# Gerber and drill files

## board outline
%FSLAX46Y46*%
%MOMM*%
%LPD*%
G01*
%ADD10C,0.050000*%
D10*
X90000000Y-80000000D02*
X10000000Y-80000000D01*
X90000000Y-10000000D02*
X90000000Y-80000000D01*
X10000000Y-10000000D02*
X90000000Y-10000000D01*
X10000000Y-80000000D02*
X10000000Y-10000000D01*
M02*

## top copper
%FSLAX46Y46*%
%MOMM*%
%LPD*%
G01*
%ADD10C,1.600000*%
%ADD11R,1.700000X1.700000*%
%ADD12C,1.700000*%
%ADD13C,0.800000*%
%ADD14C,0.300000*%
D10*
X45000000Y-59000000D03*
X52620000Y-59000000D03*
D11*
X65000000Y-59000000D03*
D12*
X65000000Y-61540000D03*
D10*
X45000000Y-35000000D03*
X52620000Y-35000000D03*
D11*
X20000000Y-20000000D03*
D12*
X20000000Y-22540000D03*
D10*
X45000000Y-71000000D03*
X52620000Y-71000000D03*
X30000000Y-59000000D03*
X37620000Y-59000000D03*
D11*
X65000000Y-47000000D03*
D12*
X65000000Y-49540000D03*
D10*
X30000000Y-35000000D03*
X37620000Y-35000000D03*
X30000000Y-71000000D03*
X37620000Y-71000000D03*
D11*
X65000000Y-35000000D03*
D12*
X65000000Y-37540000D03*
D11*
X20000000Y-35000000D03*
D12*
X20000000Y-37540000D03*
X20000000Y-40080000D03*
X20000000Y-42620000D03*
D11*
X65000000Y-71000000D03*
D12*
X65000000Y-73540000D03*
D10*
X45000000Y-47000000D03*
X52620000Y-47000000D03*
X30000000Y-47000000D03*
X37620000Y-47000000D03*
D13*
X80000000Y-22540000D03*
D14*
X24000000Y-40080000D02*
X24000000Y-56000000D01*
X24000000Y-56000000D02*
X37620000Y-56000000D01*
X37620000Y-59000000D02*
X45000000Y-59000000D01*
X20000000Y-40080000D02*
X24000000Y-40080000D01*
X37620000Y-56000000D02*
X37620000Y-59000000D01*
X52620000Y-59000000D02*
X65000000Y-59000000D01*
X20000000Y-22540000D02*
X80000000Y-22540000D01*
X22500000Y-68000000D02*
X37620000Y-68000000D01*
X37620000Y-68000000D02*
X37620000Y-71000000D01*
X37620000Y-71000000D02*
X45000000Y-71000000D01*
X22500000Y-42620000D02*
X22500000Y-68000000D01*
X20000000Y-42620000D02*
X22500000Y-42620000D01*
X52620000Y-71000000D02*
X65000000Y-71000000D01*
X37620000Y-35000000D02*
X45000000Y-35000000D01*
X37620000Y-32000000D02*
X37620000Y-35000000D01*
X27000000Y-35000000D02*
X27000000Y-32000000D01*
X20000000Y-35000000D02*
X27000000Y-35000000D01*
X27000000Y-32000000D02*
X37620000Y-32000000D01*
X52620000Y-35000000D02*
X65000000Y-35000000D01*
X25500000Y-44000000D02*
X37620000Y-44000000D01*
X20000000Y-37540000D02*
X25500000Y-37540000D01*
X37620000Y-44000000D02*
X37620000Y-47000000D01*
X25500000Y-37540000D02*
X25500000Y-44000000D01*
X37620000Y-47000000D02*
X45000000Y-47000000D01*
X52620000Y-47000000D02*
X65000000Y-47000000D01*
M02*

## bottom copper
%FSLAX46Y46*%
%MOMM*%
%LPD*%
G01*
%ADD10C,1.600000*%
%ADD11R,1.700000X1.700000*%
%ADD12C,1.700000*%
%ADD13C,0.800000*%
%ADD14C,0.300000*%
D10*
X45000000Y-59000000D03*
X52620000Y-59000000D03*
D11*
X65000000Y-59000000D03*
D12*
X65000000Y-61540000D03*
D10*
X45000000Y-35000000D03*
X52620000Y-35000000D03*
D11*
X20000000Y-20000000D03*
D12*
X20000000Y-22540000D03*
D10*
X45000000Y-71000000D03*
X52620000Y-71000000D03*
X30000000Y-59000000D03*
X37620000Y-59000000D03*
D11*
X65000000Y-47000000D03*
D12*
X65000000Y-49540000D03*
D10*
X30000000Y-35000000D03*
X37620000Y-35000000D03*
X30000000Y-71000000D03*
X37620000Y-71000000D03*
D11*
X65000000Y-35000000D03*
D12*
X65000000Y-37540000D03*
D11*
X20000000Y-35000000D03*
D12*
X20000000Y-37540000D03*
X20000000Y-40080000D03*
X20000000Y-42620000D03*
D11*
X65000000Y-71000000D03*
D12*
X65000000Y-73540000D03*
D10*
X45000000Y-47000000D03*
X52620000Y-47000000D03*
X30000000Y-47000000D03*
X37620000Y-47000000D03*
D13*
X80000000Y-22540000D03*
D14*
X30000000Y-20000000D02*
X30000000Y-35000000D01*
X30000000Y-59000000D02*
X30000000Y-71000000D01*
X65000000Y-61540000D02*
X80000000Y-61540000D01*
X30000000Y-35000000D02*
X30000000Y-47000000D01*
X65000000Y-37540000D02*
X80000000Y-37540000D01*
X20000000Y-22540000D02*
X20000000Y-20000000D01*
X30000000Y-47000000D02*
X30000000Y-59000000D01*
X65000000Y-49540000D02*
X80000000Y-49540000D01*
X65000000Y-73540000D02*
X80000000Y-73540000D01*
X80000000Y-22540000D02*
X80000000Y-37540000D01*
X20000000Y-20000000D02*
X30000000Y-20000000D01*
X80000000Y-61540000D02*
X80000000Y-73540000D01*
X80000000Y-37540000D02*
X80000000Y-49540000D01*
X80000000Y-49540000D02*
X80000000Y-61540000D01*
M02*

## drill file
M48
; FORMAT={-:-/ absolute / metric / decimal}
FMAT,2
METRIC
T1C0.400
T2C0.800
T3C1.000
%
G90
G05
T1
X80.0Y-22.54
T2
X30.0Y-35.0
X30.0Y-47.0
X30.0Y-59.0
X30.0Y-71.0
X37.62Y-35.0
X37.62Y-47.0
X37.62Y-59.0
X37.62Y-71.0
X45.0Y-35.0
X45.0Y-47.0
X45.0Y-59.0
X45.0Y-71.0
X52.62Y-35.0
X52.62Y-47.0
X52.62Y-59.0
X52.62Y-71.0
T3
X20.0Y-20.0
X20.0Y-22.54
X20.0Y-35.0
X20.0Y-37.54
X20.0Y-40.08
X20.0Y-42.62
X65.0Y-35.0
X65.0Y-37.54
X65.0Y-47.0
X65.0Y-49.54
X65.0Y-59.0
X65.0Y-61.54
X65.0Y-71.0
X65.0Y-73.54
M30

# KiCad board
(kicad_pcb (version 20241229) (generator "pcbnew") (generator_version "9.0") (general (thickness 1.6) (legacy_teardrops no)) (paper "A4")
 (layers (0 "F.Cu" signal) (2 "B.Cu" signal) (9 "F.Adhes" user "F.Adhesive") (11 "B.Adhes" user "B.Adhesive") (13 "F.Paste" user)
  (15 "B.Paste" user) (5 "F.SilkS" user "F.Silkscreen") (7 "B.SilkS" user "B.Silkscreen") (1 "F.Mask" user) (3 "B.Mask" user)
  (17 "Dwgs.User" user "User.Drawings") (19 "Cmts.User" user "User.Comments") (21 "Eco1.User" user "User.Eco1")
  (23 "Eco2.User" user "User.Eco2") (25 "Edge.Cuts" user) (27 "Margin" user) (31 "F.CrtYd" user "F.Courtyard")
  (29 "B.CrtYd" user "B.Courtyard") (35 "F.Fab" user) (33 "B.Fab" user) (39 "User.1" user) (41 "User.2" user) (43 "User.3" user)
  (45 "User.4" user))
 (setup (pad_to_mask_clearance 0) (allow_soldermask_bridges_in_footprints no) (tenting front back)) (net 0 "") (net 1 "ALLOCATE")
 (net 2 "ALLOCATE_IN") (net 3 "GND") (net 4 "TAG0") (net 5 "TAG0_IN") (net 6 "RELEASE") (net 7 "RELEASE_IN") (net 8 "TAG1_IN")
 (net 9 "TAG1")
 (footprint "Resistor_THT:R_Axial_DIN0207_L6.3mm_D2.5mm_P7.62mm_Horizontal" (layer "F.Cu") (at 45 59)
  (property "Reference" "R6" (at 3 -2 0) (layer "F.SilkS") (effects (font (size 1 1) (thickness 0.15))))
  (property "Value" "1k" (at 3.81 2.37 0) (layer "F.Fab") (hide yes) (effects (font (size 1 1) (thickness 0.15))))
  (pad "1" thru_hole circle (at 0 0) (size 1.6 1.6) (drill 0.8) (layers "*.Cu" "*.Mask") (remove_unused_layers no) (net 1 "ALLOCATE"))
  (pad "2" thru_hole circle (at 7.62 0) (size 1.6 1.6) (drill 0.8) (layers "*.Cu" "*.Mask") (remove_unused_layers no) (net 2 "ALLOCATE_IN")))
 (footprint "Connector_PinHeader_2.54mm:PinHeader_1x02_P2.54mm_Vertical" (layer "F.Cu") (at 65 59)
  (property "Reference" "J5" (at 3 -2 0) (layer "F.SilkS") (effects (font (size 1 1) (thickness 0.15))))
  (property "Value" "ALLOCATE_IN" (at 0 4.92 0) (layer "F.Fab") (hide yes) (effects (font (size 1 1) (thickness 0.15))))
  (pad "1" thru_hole rect (at 0 0) (size 1.7 1.7) (drill 1) (layers "*.Cu" "*.Mask") (remove_unused_layers no) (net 2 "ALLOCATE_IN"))
  (pad "2" thru_hole circle (at 0 2.54) (size 1.7 1.7) (drill 1) (layers "*.Cu" "*.Mask") (remove_unused_layers no) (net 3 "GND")))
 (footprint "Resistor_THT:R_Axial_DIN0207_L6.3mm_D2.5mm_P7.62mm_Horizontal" (layer "F.Cu") (at 45 35)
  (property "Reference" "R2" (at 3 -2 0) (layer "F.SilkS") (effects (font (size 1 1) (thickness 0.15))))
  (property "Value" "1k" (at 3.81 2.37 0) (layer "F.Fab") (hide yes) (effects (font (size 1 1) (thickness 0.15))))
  (pad "1" thru_hole circle (at 0 0) (size 1.6 1.6) (drill 0.8) (layers "*.Cu" "*.Mask") (remove_unused_layers no) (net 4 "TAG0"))
  (pad "2" thru_hole circle (at 7.62 0) (size 1.6 1.6) (drill 0.8) (layers "*.Cu" "*.Mask") (remove_unused_layers no) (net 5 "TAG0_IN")))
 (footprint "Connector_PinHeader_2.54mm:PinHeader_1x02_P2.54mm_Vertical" (layer "F.Cu") (at 20 20)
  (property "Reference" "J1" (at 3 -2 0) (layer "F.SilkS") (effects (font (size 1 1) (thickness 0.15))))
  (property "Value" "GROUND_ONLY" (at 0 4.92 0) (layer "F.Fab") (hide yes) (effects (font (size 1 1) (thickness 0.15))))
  (pad "1" thru_hole rect (at 0 0) (size 1.7 1.7) (drill 1) (layers "*.Cu" "*.Mask") (remove_unused_layers no) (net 3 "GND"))
  (pad "2" thru_hole circle (at 0 2.54) (size 1.7 1.7) (drill 1) (layers "*.Cu" "*.Mask") (remove_unused_layers no) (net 3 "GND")))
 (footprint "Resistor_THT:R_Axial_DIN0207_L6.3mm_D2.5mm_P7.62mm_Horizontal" (layer "F.Cu") (at 45 71)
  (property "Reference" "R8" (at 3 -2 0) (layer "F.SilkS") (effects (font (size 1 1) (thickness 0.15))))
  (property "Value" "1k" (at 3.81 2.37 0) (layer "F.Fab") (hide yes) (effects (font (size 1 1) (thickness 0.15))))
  (pad "1" thru_hole circle (at 0 0) (size 1.6 1.6) (drill 0.8) (layers "*.Cu" "*.Mask") (remove_unused_layers no) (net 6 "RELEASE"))
  (pad "2" thru_hole circle (at 7.62 0) (size 1.6 1.6) (drill 0.8) (layers "*.Cu" "*.Mask") (remove_unused_layers no) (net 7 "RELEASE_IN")))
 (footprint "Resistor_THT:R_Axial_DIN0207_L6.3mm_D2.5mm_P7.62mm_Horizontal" (layer "F.Cu") (at 30 59)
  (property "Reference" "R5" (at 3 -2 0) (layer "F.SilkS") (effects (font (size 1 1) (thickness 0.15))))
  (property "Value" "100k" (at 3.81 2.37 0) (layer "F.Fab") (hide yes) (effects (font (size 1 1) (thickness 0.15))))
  (pad "1" thru_hole circle (at 0 0) (size 1.6 1.6) (drill 0.8) (layers "*.Cu" "*.Mask") (remove_unused_layers no) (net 3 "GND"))
  (pad "2" thru_hole circle (at 7.62 0) (size 1.6 1.6) (drill 0.8) (layers "*.Cu" "*.Mask") (remove_unused_layers no) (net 1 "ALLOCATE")))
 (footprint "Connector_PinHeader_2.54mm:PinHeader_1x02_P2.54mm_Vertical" (layer "F.Cu") (at 65 47)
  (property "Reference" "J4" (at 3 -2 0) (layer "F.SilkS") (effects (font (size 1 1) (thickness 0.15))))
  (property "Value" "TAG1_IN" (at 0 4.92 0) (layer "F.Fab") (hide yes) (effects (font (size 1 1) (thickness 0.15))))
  (pad "1" thru_hole rect (at 0 0) (size 1.7 1.7) (drill 1) (layers "*.Cu" "*.Mask") (remove_unused_layers no) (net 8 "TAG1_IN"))
  (pad "2" thru_hole circle (at 0 2.54) (size 1.7 1.7) (drill 1) (layers "*.Cu" "*.Mask") (remove_unused_layers no) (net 3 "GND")))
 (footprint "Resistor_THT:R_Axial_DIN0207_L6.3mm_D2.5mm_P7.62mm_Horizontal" (layer "F.Cu") (at 30 35)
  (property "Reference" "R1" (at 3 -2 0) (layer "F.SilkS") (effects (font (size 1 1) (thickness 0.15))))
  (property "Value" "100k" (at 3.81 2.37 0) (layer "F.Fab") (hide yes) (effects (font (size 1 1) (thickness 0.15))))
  (pad "1" thru_hole circle (at 0 0) (size 1.6 1.6) (drill 0.8) (layers "*.Cu" "*.Mask") (remove_unused_layers no) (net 3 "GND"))
  (pad "2" thru_hole circle (at 7.62 0) (size 1.6 1.6) (drill 0.8) (layers "*.Cu" "*.Mask") (remove_unused_layers no) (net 4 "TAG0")))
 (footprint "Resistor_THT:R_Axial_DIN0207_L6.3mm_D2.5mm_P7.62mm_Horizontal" (layer "F.Cu") (at 30 71)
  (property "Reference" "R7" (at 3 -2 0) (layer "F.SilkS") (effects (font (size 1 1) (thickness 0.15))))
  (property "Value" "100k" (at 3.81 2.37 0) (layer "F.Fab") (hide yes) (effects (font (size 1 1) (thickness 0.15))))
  (pad "1" thru_hole circle (at 0 0) (size 1.6 1.6) (drill 0.8) (layers "*.Cu" "*.Mask") (remove_unused_layers no) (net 3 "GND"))
  (pad "2" thru_hole circle (at 7.62 0) (size 1.6 1.6) (drill 0.8) (layers "*.Cu" "*.Mask") (remove_unused_layers no) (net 6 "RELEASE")))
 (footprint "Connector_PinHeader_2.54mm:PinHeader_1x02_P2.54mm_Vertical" (layer "F.Cu") (at 65 35)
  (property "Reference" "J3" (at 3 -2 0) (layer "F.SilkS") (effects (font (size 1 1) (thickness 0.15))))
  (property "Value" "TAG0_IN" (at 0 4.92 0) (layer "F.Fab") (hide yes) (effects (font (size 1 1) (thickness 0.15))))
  (pad "1" thru_hole rect (at 0 0) (size 1.7 1.7) (drill 1) (layers "*.Cu" "*.Mask") (remove_unused_layers no) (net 5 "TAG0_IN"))
  (pad "2" thru_hole circle (at 0 2.54) (size 1.7 1.7) (drill 1) (layers "*.Cu" "*.Mask") (remove_unused_layers no) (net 3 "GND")))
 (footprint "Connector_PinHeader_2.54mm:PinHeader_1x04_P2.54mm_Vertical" (layer "F.Cu") (at 20 35)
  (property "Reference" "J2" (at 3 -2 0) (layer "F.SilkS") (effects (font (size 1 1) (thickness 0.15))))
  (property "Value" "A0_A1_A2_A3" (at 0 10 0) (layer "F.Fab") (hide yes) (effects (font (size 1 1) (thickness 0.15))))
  (pad "1" thru_hole rect (at 0 0) (size 1.7 1.7) (drill 1) (layers "*.Cu" "*.Mask") (remove_unused_layers no) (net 4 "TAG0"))
  (pad "2" thru_hole circle (at 0 2.54) (size 1.7 1.7) (drill 1) (layers "*.Cu" "*.Mask") (remove_unused_layers no) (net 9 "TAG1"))
  (pad "3" thru_hole circle (at 0 5.08) (size 1.7 1.7) (drill 1) (layers "*.Cu" "*.Mask") (remove_unused_layers no) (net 1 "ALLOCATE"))
  (pad "4" thru_hole circle (at 0 7.62) (size 1.7 1.7) (drill 1) (layers "*.Cu" "*.Mask") (remove_unused_layers no) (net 6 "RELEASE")))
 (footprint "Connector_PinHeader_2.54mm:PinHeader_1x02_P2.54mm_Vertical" (layer "F.Cu") (at 65 71)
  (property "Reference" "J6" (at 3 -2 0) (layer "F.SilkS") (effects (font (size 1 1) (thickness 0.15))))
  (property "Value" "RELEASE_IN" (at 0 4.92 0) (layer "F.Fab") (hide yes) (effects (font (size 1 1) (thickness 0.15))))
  (pad "1" thru_hole rect (at 0 0) (size 1.7 1.7) (drill 1) (layers "*.Cu" "*.Mask") (remove_unused_layers no) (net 7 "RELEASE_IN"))
  (pad "2" thru_hole circle (at 0 2.54) (size 1.7 1.7) (drill 1) (layers "*.Cu" "*.Mask") (remove_unused_layers no) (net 3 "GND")))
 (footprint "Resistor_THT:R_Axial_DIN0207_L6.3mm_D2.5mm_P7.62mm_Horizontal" (layer "F.Cu") (at 45 47)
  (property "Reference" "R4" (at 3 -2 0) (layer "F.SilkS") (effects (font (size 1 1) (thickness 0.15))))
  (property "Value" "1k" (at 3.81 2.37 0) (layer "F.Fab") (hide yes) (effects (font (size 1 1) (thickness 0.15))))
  (pad "1" thru_hole circle (at 0 0) (size 1.6 1.6) (drill 0.8) (layers "*.Cu" "*.Mask") (remove_unused_layers no) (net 9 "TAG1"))
  (pad "2" thru_hole circle (at 7.62 0) (size 1.6 1.6) (drill 0.8) (layers "*.Cu" "*.Mask") (remove_unused_layers no) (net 8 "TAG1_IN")))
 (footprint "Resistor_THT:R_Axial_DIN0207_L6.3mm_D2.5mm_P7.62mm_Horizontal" (layer "F.Cu") (at 30 47)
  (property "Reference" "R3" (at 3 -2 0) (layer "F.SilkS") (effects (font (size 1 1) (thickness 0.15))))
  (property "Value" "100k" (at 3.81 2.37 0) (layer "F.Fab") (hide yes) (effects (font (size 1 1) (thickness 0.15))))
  (pad "1" thru_hole circle (at 0 0) (size 1.6 1.6) (drill 0.8) (layers "*.Cu" "*.Mask") (remove_unused_layers no) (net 3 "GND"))
  (pad "2" thru_hole circle (at 7.62 0) (size 1.6 1.6) (drill 0.8) (layers "*.Cu" "*.Mask") (remove_unused_layers no) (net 9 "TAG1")))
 (gr_line (start 90 80) (end 10 80) (stroke (width 0.05) (type default)) (layer "Edge.Cuts"))
 (gr_line (start 90 10) (end 90 80) (stroke (width 0.05) (type default)) (layer "Edge.Cuts"))
 (gr_line (start 10 10) (end 90 10) (stroke (width 0.05) (type default)) (layer "Edge.Cuts"))
 (gr_line (start 10 80) (end 10 10) (stroke (width 0.05) (type default)) (layer "Edge.Cuts"))
 (segment (start 24 40.08) (end 24 56) (width 0.3) (layer "F.Cu") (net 1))
 (segment (start 24 56) (end 37.62 56) (width 0.3) (layer "F.Cu") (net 1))
 (segment (start 37.62 59) (end 45 59) (width 0.3) (layer "F.Cu") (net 1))
 (segment (start 20 40.08) (end 24 40.08) (width 0.3) (layer "F.Cu") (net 1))
 (segment (start 37.62 56) (end 37.62 59) (width 0.3) (layer "F.Cu") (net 1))
 (segment (start 52.62 59) (end 65 59) (width 0.3) (layer "F.Cu") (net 2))
 (segment (start 20 22.54) (end 80 22.54) (width 0.3) (layer "F.Cu") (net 3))
 (via (at 80 22.54) (size 0.8) (drill 0.4) (layers "F.Cu" "B.Cu") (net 3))
 (segment (start 30 20) (end 30 35) (width 0.3) (layer "B.Cu") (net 3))
 (segment (start 30 59) (end 30 71) (width 0.3) (layer "B.Cu") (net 3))
 (segment (start 65 61.54) (end 80 61.54) (width 0.3) (layer "B.Cu") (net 3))
 (segment (start 30 35) (end 30 47) (width 0.3) (layer "B.Cu") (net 3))
 (segment (start 65 37.54) (end 80 37.54) (width 0.3) (layer "B.Cu") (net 3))
 (segment (start 20 22.54) (end 20 20) (width 0.3) (layer "B.Cu") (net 3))
 (segment (start 30 47) (end 30 59) (width 0.3) (layer "B.Cu") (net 3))
 (segment (start 65 49.54) (end 80 49.54) (width 0.3) (layer "B.Cu") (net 3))
 (segment (start 65 73.54) (end 80 73.54) (width 0.3) (layer "B.Cu") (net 3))
 (segment (start 80 22.54) (end 80 37.54) (width 0.3) (layer "B.Cu") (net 3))
 (segment (start 20 20) (end 30 20) (width 0.3) (layer "B.Cu") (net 3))
 (segment (start 80 61.54) (end 80 73.54) (width 0.3) (layer "B.Cu") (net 3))
 (segment (start 80 37.54) (end 80 49.54) (width 0.3) (layer "B.Cu") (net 3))
 (segment (start 80 49.54) (end 80 61.54) (width 0.3) (layer "B.Cu") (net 3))
 (segment (start 22.5 68) (end 37.62 68) (width 0.3) (layer "F.Cu") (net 6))
 (segment (start 37.62 68) (end 37.62 71) (width 0.3) (layer "F.Cu") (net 6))
 (segment (start 37.62 71) (end 45 71) (width 0.3) (layer "F.Cu") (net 6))
 (segment (start 22.5 42.62) (end 22.5 68) (width 0.3) (layer "F.Cu") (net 6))
 (segment (start 20 42.62) (end 22.5 42.62) (width 0.3) (layer "F.Cu") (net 6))
 (segment (start 52.62 71) (end 65 71) (width 0.3) (layer "F.Cu") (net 7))
 (segment (start 37.62 35) (end 45 35) (width 0.3) (layer "F.Cu") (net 4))
 (segment (start 37.62 32) (end 37.62 35) (width 0.3) (layer "F.Cu") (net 4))
 (segment (start 27 35) (end 27 32) (width 0.3) (layer "F.Cu") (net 4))
 (segment (start 20 35) (end 27 35) (width 0.3) (layer "F.Cu") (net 4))
 (segment (start 27 32) (end 37.62 32) (width 0.3) (layer "F.Cu") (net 4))
 (segment (start 52.62 35) (end 65 35) (width 0.3) (layer "F.Cu") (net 5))
 (segment (start 25.5 44) (end 37.62 44) (width 0.3) (layer "F.Cu") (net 9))
 (segment (start 20 37.54) (end 25.5 37.54) (width 0.3) (layer "F.Cu") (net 9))
 (segment (start 37.62 44) (end 37.62 47) (width 0.3) (layer "F.Cu") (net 9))
 (segment (start 25.5 37.54) (end 25.5 44) (width 0.3) (layer "F.Cu") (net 9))
 (segment (start 37.62 47) (end 45 47) (width 0.3) (layer "F.Cu") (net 9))
 (segment (start 52.62 47) (end 65 47) (width 0.3) (layer "F.Cu") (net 8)))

